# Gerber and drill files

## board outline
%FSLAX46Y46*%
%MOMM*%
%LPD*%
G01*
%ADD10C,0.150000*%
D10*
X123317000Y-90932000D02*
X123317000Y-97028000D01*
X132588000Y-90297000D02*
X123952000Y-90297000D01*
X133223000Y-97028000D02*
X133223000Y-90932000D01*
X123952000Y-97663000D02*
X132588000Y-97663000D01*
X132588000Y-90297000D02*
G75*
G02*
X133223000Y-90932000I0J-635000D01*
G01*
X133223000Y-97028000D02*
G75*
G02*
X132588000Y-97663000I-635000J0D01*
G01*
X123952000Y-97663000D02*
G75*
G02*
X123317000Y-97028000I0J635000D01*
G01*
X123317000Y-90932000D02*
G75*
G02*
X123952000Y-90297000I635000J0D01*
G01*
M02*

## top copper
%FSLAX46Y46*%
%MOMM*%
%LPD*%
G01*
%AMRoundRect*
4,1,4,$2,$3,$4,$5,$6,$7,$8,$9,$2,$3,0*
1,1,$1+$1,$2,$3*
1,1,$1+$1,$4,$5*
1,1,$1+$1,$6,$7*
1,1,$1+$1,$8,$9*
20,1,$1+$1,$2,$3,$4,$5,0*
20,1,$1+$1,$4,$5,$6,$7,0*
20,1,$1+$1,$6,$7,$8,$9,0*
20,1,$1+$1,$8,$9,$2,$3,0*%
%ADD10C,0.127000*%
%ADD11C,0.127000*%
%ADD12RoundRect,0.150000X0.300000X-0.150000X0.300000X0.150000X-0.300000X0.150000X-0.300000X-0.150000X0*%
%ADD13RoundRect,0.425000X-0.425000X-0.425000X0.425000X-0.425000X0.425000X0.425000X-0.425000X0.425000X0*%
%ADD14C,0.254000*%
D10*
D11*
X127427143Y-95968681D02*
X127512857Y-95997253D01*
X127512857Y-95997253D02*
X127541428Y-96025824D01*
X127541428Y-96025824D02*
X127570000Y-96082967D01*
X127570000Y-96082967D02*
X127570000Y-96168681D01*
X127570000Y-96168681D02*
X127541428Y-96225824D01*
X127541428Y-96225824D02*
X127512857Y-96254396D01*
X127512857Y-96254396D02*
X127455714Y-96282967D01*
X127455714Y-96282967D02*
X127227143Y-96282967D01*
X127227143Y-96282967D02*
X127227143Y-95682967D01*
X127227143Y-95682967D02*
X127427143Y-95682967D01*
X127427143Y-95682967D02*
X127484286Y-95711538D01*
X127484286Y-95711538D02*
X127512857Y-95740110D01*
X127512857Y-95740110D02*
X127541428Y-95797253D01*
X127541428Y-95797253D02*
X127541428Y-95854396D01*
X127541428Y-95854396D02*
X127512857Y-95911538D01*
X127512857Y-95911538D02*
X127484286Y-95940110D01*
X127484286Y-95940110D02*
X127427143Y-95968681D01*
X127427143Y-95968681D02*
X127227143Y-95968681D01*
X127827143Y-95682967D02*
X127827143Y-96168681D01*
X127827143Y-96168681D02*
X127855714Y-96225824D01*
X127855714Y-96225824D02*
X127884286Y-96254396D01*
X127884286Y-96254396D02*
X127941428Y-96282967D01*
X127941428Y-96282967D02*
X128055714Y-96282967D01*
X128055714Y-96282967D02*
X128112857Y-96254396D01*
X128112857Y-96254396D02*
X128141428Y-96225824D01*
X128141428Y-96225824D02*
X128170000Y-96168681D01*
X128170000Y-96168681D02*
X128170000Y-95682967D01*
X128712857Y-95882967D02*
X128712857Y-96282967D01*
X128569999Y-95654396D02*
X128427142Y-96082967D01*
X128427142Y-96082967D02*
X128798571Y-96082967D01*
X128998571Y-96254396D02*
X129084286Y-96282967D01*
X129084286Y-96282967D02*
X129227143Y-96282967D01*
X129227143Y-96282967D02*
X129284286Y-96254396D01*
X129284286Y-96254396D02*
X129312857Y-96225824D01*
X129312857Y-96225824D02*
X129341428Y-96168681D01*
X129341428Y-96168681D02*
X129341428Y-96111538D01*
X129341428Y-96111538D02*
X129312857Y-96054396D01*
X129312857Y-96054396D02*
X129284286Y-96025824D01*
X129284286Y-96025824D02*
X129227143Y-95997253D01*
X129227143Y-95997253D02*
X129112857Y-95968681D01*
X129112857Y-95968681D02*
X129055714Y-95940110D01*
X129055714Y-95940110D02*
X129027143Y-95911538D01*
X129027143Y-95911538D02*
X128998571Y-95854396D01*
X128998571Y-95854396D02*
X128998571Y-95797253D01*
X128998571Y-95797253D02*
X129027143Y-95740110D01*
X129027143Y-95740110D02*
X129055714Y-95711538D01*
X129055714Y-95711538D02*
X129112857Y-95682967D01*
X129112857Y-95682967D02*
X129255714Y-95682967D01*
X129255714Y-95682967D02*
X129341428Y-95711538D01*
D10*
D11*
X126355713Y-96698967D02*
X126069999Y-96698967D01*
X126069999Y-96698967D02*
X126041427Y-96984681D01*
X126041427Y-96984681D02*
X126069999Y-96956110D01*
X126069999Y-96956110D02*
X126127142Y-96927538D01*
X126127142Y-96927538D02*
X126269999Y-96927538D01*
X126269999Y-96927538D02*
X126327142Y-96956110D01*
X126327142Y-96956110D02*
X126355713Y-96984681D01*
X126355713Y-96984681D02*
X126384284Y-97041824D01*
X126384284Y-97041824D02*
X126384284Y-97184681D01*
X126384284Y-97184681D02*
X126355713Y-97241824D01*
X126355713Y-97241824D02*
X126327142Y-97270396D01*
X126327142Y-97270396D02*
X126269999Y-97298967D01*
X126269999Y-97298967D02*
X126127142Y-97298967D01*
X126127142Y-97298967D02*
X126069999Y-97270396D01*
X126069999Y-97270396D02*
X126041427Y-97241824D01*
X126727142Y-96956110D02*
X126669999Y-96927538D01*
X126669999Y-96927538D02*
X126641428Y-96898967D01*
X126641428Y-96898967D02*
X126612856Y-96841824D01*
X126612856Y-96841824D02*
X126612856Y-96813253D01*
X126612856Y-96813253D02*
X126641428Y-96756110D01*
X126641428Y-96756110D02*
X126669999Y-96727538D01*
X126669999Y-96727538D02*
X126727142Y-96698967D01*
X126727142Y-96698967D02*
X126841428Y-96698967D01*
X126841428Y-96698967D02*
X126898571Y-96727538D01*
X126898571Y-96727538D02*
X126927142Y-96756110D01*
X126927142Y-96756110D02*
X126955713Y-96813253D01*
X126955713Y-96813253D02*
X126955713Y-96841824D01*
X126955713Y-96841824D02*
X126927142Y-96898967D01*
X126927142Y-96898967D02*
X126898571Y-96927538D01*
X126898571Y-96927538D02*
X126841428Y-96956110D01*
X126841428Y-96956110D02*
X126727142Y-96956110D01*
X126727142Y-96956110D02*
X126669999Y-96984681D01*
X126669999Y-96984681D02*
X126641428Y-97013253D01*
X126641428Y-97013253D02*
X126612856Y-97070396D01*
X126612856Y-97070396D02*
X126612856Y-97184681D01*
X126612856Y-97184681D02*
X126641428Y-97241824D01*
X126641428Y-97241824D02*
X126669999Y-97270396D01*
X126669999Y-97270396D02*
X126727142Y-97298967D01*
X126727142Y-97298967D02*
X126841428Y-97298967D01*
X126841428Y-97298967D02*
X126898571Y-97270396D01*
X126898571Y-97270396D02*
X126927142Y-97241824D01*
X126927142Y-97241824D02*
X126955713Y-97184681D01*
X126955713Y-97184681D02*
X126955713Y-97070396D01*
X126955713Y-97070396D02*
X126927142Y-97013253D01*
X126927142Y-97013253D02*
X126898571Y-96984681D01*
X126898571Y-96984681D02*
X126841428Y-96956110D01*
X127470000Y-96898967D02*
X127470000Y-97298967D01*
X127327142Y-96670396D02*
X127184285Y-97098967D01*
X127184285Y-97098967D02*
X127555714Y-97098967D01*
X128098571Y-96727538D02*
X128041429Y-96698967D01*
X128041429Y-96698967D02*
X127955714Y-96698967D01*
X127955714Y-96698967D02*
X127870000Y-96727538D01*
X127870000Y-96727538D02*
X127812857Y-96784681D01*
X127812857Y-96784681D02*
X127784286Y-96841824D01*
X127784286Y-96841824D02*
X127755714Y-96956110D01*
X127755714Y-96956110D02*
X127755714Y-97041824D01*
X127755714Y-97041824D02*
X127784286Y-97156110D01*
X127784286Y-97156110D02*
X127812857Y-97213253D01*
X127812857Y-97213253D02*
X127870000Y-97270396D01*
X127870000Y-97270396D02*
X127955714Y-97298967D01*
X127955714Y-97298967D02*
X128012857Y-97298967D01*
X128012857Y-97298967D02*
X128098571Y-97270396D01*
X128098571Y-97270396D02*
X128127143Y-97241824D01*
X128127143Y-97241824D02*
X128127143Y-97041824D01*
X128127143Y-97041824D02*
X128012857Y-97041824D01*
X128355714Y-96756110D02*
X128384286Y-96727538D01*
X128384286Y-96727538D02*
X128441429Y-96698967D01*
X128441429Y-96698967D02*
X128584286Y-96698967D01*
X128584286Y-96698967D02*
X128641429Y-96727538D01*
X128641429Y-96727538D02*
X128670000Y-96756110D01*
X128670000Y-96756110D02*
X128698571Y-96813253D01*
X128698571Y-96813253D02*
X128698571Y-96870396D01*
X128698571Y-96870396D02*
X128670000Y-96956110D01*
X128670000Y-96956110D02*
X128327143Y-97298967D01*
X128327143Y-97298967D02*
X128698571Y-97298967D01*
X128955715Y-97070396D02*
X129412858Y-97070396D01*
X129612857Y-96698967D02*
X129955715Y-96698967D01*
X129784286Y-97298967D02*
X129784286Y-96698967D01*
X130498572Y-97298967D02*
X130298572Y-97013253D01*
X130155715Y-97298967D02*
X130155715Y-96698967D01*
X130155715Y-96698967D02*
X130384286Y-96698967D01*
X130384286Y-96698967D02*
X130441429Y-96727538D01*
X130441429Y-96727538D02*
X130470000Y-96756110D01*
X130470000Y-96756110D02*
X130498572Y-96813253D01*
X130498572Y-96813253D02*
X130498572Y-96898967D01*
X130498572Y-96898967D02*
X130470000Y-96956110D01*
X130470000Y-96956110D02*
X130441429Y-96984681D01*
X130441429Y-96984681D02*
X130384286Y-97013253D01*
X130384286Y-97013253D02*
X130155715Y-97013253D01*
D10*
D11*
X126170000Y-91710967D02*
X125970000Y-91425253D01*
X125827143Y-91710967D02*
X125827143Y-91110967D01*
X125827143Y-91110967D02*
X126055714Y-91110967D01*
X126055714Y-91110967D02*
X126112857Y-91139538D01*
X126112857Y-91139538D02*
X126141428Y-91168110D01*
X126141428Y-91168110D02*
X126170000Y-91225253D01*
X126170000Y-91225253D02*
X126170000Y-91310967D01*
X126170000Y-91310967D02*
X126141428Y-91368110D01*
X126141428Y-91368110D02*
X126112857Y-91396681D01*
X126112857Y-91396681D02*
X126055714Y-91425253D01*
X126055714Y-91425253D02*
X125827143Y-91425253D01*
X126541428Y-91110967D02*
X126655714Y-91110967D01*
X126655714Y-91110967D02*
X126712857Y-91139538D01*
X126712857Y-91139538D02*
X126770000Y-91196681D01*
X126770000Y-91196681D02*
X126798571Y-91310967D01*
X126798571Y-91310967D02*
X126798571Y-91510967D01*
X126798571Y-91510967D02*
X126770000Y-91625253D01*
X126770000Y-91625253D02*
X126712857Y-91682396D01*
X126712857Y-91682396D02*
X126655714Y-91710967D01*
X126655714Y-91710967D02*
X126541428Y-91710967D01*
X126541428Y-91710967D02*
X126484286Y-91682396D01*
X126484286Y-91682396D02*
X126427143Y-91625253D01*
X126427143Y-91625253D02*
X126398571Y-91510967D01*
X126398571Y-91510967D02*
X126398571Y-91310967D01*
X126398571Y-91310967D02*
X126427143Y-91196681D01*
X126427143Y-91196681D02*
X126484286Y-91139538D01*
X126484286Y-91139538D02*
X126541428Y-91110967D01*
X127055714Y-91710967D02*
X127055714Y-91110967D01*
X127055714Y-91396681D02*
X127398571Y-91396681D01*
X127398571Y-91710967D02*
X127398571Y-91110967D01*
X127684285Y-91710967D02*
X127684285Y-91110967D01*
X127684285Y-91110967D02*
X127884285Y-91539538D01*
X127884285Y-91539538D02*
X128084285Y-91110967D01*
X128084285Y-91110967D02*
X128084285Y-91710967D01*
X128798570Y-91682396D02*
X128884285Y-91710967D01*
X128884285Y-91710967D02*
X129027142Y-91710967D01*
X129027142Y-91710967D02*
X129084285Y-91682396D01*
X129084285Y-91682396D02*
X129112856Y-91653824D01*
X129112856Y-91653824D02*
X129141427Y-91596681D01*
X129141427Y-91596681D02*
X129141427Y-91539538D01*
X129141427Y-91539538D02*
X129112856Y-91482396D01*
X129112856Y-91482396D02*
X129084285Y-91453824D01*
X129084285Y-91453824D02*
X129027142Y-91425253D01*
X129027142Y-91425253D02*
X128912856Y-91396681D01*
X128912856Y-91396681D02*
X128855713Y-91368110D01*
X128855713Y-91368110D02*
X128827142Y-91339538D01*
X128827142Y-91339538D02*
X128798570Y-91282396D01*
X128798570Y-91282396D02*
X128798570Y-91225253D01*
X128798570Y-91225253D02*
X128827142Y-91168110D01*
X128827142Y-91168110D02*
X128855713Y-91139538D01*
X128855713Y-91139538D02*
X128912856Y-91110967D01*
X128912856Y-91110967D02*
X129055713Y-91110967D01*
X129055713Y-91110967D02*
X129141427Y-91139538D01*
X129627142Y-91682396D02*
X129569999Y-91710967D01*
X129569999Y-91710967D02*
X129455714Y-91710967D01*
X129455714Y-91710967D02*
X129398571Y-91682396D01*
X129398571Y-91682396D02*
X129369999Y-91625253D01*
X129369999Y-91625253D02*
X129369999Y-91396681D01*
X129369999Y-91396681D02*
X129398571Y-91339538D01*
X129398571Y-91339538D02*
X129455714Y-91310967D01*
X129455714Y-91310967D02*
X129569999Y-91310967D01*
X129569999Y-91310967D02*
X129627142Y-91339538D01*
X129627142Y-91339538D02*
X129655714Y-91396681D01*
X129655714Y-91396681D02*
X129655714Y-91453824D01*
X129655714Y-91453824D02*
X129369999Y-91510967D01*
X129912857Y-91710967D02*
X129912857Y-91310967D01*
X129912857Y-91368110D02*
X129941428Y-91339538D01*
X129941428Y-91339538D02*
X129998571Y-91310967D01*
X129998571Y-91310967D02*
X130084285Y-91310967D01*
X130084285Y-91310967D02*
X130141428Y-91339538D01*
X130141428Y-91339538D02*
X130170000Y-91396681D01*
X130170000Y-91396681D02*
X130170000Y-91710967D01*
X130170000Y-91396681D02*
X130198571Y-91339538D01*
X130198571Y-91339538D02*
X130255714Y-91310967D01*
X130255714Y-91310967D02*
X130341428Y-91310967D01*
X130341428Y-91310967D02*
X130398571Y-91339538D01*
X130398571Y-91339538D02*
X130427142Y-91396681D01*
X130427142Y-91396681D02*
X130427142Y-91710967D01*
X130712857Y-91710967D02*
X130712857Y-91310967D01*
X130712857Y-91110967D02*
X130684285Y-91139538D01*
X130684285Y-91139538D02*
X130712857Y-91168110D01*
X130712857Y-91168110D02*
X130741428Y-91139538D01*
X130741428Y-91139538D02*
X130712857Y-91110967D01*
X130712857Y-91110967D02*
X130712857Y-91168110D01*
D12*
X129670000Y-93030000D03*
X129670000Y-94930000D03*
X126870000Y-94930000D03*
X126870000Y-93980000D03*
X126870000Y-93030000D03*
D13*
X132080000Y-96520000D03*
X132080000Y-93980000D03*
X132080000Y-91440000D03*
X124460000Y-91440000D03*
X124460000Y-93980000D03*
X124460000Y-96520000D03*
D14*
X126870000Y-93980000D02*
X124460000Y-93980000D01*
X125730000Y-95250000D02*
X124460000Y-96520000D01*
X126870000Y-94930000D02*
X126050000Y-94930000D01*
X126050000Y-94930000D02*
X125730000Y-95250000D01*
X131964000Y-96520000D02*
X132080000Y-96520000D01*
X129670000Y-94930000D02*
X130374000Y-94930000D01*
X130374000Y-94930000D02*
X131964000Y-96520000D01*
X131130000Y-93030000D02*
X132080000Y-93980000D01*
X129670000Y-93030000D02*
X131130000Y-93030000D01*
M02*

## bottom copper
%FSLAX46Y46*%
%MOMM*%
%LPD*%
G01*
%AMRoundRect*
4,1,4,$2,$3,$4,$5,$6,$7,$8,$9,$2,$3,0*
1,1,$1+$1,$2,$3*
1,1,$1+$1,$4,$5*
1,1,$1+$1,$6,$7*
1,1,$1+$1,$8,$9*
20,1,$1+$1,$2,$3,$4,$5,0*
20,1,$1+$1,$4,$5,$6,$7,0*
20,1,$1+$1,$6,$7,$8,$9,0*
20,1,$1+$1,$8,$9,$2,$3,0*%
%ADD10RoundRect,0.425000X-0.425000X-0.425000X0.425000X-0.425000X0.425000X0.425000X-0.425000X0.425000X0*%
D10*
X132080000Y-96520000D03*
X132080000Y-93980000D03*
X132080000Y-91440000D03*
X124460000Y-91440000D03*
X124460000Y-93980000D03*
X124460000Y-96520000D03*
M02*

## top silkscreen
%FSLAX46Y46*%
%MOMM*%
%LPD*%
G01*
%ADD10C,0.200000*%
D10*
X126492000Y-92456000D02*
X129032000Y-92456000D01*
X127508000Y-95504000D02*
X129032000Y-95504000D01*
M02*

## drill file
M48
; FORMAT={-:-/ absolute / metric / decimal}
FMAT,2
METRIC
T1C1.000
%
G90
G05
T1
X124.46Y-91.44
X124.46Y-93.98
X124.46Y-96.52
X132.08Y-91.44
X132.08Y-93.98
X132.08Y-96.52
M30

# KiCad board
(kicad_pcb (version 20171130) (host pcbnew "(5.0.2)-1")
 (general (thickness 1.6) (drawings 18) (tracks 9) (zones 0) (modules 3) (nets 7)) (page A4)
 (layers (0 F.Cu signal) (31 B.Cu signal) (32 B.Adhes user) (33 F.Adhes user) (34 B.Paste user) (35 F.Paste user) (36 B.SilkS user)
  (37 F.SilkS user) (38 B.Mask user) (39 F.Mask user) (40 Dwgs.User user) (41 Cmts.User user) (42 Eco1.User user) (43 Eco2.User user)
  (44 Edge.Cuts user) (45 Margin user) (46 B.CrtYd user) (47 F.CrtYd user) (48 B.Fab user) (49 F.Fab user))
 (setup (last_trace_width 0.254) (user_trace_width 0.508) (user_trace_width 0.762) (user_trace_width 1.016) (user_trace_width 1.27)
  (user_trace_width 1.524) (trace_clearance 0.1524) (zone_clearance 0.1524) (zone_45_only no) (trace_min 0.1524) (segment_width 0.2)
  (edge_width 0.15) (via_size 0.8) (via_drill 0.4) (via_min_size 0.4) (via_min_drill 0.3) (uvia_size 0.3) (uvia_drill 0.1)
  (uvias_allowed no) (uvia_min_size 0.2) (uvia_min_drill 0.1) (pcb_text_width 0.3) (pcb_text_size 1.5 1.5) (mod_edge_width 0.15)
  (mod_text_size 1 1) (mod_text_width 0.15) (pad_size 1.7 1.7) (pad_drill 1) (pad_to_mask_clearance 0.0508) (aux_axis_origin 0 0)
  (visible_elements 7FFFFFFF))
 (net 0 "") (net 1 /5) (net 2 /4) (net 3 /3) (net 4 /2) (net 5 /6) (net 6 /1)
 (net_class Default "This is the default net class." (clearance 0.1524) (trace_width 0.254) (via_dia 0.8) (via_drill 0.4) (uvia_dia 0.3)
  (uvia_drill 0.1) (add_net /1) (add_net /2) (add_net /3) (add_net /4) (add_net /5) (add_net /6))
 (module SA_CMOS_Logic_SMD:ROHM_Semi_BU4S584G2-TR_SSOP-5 (layer F.Cu) (at 128.27 93.98)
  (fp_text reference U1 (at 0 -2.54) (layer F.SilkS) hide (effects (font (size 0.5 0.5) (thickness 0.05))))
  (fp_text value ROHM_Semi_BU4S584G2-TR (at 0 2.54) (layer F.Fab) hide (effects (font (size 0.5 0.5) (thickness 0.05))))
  (fp_line (start -1.778 -1.524) (end 0.762 -1.524) (layer F.SilkS) (width 0.2))
  (fp_line (start -0.762 1.524) (end 0.762 1.524) (layer F.SilkS) (width 0.2))
  (pad 5 smd roundrect (at 1.4 -0.95 90) (size 0.6 0.9) (layers F.Cu F.Paste F.Mask) (roundrect_rratio 0.25) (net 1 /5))
  (pad 4 smd roundrect (at 1.4 0.95 90) (size 0.6 0.9) (layers F.Cu F.Paste F.Mask) (roundrect_rratio 0.25) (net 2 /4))
  (pad 3 smd roundrect (at -1.4 0.95 90) (size 0.6 0.9) (layers F.Cu F.Paste F.Mask) (roundrect_rratio 0.25) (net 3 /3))
  (pad 2 smd roundrect (at -1.4 0 90) (size 0.6 0.9) (layers F.Cu F.Paste F.Mask) (roundrect_rratio 0.25) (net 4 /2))
  (pad 1 smd roundrect (at -1.4 -0.95 90) (size 0.6 0.9) (layers F.Cu F.Paste F.Mask) (roundrect_rratio 0.25)))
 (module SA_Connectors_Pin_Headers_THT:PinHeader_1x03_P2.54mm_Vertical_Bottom (layer F.Cu) (at 132.08 91.44)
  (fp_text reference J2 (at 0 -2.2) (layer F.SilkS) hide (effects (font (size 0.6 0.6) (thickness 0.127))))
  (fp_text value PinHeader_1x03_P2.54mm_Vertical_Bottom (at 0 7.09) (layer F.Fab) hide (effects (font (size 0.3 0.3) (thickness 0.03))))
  (pad 3 thru_hole roundrect (at 0 5.08) (size 1.7 1.7) (drill 1) (layers *.Cu *.Mask) (roundrect_rratio 0.25) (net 2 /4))
  (pad 2 thru_hole roundrect (at 0 2.54) (size 1.7 1.7) (drill 1) (layers *.Cu *.Mask) (roundrect_rratio 0.25) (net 1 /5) (zone_connect 2))
  (pad 1 thru_hole roundrect (at 0 0) (size 1.7 1.7) (drill 1) (layers *.Cu *.Mask) (roundrect_rratio 0.25) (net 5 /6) (zone_connect 2)))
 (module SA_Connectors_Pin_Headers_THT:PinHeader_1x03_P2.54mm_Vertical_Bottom (layer F.Cu) (at 124.46 91.44)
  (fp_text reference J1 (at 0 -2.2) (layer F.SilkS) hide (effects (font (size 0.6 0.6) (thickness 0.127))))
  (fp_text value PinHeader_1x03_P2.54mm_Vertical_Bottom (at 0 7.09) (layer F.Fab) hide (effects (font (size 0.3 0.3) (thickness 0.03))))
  (pad 1 thru_hole roundrect (at 0 0) (size 1.7 1.7) (drill 1) (layers *.Cu *.Mask) (roundrect_rratio 0.25) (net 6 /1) (zone_connect 2))
  (pad 2 thru_hole roundrect (at 0 2.54) (size 1.7 1.7) (drill 1) (layers *.Cu *.Mask) (roundrect_rratio 0.25) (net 4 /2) (zone_connect 2))
  (pad 3 thru_hole roundrect (at 0 5.08) (size 1.7 1.7) (drill 1) (layers *.Cu *.Mask) (roundrect_rratio 0.25) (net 3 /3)))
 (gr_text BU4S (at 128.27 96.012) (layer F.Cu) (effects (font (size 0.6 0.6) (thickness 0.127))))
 (gr_line (start 123.317 90.932) (end 123.317 97.028) (layer Edge.Cuts) (width 0.15))
 (gr_line (start 132.588 90.297) (end 123.952 90.297) (layer Edge.Cuts) (width 0.15))
 (gr_line (start 133.223 97.028) (end 133.223 90.932) (layer Edge.Cuts) (width 0.15))
 (gr_line (start 123.952 97.663) (end 132.588 97.663) (layer Edge.Cuts) (width 0.15))
 (gr_arc (start 132.588 90.932) (end 133.223 90.932) (angle -90) (layer Edge.Cuts) (width 0.15))
 (gr_arc (start 132.588 97.028) (end 132.588 97.663) (angle -90) (layer Edge.Cuts) (width 0.15))
 (gr_arc (start 123.952 97.028) (end 123.317 97.028) (angle -90) (layer Edge.Cuts) (width 0.15))
 (gr_arc (start 123.952 90.932) (end 123.952 90.297) (angle -90) (layer Edge.Cuts) (width 0.15))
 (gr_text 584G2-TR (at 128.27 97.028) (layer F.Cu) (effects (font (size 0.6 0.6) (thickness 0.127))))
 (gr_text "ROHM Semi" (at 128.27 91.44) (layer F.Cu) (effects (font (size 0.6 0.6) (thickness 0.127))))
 (segment (start 126.87 93.98) (end 124.46 93.98) (width 0.254) (layer F.Cu) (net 4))
 (segment (start 125.73 95.25) (end 124.46 96.52) (width 0.254) (layer F.Cu) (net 3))
 (segment (start 126.87 94.93) (end 126.05 94.93) (width 0.254) (layer F.Cu) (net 3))
 (segment (start 126.05 94.93) (end 125.73 95.25) (width 0.254) (layer F.Cu) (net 3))
 (segment (start 131.964 96.52) (end 132.08 96.52) (width 0.254) (layer F.Cu) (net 2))
 (segment (start 129.67 94.93) (end 130.374 94.93) (width 0.254) (layer F.Cu) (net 2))
 (segment (start 130.374 94.93) (end 131.964 96.52) (width 0.254) (layer F.Cu) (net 2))
 (segment (start 131.13 93.03) (end 132.08 93.98) (width 0.254) (layer F.Cu) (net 1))
 (segment (start 129.67 93.03) (end 131.13 93.03) (width 0.254) (layer F.Cu) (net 1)))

